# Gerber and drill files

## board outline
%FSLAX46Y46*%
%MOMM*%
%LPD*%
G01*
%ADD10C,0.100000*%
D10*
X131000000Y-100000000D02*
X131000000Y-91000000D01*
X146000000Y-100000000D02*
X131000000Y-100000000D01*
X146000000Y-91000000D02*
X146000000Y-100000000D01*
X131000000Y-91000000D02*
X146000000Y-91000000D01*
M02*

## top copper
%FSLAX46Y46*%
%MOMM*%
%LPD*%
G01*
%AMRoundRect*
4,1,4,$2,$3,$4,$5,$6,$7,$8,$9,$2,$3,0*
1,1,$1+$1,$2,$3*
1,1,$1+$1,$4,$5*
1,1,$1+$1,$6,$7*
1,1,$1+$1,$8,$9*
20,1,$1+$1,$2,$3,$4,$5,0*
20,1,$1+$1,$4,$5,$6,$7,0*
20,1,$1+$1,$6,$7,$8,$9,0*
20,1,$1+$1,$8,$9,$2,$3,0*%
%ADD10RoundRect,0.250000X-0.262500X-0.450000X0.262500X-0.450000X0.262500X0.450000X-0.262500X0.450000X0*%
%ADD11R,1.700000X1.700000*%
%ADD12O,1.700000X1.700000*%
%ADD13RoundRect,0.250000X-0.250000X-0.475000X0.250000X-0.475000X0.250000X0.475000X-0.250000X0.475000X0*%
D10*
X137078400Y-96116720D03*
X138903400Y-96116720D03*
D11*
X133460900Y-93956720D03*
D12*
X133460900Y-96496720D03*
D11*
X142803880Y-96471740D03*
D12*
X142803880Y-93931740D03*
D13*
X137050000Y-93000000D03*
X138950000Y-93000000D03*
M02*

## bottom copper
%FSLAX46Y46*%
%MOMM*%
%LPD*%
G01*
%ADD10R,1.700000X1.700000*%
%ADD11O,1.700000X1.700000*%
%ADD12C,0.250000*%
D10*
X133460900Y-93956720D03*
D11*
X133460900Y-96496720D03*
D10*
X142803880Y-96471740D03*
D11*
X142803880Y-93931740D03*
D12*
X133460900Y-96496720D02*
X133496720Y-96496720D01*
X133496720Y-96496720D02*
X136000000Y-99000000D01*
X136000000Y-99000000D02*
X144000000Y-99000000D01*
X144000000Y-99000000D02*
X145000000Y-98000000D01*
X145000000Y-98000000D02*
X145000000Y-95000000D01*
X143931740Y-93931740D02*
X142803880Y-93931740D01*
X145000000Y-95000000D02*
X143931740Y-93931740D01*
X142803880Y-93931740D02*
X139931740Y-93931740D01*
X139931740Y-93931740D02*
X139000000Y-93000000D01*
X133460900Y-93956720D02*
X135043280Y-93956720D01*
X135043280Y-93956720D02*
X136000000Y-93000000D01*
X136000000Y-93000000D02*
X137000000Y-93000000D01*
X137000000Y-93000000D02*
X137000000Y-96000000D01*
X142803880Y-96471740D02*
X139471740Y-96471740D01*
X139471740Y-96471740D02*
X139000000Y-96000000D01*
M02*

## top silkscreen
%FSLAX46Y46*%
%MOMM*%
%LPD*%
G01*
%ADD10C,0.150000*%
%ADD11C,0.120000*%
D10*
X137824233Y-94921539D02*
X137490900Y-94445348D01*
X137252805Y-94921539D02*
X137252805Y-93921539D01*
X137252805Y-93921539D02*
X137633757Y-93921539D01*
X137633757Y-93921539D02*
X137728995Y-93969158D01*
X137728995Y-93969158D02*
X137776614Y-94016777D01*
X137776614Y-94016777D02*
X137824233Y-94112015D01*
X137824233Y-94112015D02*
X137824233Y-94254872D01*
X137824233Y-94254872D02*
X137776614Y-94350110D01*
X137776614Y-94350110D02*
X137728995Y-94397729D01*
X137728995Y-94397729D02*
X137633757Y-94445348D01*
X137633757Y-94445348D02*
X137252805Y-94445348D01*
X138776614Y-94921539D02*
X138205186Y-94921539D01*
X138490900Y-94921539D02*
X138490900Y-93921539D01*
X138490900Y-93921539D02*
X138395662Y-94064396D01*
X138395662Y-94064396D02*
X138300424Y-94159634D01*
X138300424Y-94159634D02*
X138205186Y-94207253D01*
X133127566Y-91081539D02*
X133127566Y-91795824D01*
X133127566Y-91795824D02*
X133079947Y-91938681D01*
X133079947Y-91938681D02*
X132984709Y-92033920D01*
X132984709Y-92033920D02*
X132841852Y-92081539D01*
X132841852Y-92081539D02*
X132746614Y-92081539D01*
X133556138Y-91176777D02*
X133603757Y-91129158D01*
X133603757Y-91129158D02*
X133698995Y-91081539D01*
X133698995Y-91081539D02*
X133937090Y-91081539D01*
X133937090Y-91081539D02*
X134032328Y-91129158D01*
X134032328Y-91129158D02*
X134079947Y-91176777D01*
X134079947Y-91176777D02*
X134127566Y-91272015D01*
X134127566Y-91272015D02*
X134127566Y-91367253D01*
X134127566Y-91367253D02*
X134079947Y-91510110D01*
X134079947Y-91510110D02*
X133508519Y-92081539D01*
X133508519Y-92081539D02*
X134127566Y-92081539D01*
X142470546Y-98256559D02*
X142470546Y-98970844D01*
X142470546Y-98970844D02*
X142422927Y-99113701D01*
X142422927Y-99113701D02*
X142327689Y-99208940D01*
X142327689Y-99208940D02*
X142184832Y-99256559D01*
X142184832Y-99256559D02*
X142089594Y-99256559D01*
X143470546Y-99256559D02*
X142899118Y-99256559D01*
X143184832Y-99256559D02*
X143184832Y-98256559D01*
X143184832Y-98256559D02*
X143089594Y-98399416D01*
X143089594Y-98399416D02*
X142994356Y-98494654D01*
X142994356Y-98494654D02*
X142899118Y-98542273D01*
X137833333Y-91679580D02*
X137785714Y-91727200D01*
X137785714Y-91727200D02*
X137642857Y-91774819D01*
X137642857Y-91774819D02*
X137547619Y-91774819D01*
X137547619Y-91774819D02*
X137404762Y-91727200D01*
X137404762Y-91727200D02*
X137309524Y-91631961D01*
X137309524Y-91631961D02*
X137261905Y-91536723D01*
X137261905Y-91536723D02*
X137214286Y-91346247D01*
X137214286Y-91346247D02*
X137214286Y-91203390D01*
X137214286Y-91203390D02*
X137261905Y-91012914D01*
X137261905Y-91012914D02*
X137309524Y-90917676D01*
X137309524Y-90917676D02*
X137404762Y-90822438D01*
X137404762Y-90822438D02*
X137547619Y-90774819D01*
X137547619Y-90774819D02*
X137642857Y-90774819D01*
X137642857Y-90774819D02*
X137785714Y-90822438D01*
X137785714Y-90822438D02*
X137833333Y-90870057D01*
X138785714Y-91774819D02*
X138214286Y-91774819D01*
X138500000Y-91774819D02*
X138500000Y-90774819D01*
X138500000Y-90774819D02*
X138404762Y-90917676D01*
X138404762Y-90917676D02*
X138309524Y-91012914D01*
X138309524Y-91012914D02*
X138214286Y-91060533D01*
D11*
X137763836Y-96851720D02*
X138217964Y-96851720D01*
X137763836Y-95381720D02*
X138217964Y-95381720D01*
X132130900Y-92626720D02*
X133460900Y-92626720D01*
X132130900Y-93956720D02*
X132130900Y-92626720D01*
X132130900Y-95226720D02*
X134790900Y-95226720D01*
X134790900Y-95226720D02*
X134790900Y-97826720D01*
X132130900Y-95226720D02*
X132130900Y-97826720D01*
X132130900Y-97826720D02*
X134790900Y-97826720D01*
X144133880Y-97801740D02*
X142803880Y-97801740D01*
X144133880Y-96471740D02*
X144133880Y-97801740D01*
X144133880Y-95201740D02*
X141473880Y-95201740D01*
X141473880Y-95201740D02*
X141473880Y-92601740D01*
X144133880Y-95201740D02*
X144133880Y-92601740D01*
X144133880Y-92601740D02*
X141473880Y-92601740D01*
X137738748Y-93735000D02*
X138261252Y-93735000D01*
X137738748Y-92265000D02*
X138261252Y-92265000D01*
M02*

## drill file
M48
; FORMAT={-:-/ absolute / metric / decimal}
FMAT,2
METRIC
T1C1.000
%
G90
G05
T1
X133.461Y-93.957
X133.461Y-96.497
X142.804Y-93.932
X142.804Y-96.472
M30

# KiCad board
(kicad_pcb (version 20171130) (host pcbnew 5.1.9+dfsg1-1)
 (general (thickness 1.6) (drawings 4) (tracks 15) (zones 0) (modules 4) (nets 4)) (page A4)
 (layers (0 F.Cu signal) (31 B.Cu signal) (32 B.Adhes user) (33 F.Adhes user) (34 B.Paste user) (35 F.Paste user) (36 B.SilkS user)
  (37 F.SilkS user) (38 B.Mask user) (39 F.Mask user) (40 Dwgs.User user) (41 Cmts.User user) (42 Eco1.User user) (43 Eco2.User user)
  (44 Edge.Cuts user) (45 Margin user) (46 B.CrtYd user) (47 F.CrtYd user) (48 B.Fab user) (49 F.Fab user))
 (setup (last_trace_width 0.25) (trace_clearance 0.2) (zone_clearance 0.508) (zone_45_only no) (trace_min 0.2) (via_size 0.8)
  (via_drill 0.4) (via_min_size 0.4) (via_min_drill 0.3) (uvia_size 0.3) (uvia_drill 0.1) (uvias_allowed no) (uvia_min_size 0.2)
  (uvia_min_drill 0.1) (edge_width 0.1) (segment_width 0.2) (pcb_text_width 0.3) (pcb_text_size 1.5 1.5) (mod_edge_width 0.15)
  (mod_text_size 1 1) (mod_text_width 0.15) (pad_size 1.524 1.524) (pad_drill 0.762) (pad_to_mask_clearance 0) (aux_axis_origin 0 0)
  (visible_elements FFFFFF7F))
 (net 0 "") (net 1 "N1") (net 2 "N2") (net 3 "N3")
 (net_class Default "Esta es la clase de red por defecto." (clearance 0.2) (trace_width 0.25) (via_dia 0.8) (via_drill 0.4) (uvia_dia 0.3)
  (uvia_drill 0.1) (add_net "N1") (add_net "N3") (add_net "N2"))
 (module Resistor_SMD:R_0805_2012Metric (layer F.Cu) (at 137.9909 96.11672)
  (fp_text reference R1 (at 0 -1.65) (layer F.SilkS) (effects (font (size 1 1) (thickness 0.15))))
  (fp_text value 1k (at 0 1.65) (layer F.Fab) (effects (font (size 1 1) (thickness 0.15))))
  (fp_line (start -0.227064 0.735) (end 0.227064 0.735) (layer F.SilkS) (width 0.12))
  (fp_line (start -0.227064 -0.735) (end 0.227064 -0.735) (layer F.SilkS) (width 0.12))
  (pad 1 smd roundrect (at -0.9125 0) (size 1.025 1.4) (layers F.Cu F.Paste F.Mask) (roundrect_rratio 0.243902) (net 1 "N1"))
  (pad 2 smd roundrect (at 0.9125 0) (size 1.025 1.4) (layers F.Cu F.Paste F.Mask) (roundrect_rratio 0.243902) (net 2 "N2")))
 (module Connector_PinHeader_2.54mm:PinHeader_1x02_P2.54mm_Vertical (layer F.Cu) (at 133.4609 93.95672)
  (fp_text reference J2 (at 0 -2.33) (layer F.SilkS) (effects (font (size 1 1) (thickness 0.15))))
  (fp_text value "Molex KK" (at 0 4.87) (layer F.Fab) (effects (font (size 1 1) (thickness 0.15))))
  (fp_line (start -1.33 -1.33) (end 0 -1.33) (layer F.SilkS) (width 0.12))
  (fp_line (start -1.33 0) (end -1.33 -1.33) (layer F.SilkS) (width 0.12))
  (fp_line (start -1.33 1.27) (end 1.33 1.27) (layer F.SilkS) (width 0.12))
  (fp_line (start 1.33 1.27) (end 1.33 3.87) (layer F.SilkS) (width 0.12))
  (fp_line (start -1.33 1.27) (end -1.33 3.87) (layer F.SilkS) (width 0.12))
  (fp_line (start -1.33 3.87) (end 1.33 3.87) (layer F.SilkS) (width 0.12))
  (pad 1 thru_hole rect (at 0 0) (size 1.7 1.7) (drill 1) (layers *.Cu *.Mask) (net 1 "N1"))
  (pad 2 thru_hole oval (at 0 2.54) (size 1.7 1.7) (drill 1) (layers *.Cu *.Mask) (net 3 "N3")))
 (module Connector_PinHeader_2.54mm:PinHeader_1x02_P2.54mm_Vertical (layer F.Cu) (at 142.80388 96.47174 180)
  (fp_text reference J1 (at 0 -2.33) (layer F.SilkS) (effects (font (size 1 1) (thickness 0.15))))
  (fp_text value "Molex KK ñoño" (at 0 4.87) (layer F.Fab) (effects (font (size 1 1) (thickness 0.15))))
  (fp_line (start -1.33 -1.33) (end 0 -1.33) (layer F.SilkS) (width 0.12))
  (fp_line (start -1.33 0) (end -1.33 -1.33) (layer F.SilkS) (width 0.12))
  (fp_line (start -1.33 1.27) (end 1.33 1.27) (layer F.SilkS) (width 0.12))
  (fp_line (start 1.33 1.27) (end 1.33 3.87) (layer F.SilkS) (width 0.12))
  (fp_line (start -1.33 1.27) (end -1.33 3.87) (layer F.SilkS) (width 0.12))
  (fp_line (start -1.33 3.87) (end 1.33 3.87) (layer F.SilkS) (width 0.12))
  (pad 1 thru_hole rect (at 0 0 180) (size 1.7 1.7) (drill 1) (layers *.Cu *.Mask) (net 2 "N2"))
  (pad 2 thru_hole oval (at 0 2.54 180) (size 1.7 1.7) (drill 1) (layers *.Cu *.Mask) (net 3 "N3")))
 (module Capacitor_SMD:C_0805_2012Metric (layer F.Cu) (at 138 93)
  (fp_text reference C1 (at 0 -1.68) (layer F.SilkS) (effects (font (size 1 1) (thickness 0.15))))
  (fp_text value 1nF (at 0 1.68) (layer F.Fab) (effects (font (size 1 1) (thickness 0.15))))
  (fp_line (start -0.261252 0.735) (end 0.261252 0.735) (layer F.SilkS) (width 0.12))
  (fp_line (start -0.261252 -0.735) (end 0.261252 -0.735) (layer F.SilkS) (width 0.12))
  (pad 1 smd roundrect (at -0.95 0) (size 1 1.45) (layers F.Cu F.Paste F.Mask) (roundrect_rratio 0.25) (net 1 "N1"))
  (pad 2 smd roundrect (at 0.95 0) (size 1 1.45) (layers F.Cu F.Paste F.Mask) (roundrect_rratio 0.25) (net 3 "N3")))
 (gr_line (start 131 100) (end 131 91) (layer Edge.Cuts) (width 0.1))
 (gr_line (start 146 100) (end 131 100) (layer Edge.Cuts) (width 0.1))
 (gr_line (start 146 91) (end 146 100) (layer Edge.Cuts) (width 0.1))
 (gr_line (start 131 91) (end 146 91) (layer Edge.Cuts) (width 0.1))
 (segment (start 133.4609 96.49672) (end 133.49672 96.49672) (width 0.25) (layer B.Cu) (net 3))
 (segment (start 133.49672 96.49672) (end 136 99) (width 0.25) (layer B.Cu) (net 3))
 (segment (start 136 99) (end 144 99) (width 0.25) (layer B.Cu) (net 3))
 (segment (start 144 99) (end 145 98) (width 0.25) (layer B.Cu) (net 3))
 (segment (start 145 98) (end 145 95) (width 0.25) (layer B.Cu) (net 3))
 (segment (start 143.93174 93.93174) (end 142.80388 93.93174) (width 0.25) (layer B.Cu) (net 3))
 (segment (start 145 95) (end 143.93174 93.93174) (width 0.25) (layer B.Cu) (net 3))
 (segment (start 142.80388 93.93174) (end 139.93174 93.93174) (width 0.25) (layer B.Cu) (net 3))
 (segment (start 139.93174 93.93174) (end 139 93) (width 0.25) (layer B.Cu) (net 3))
 (segment (start 133.4609 93.95672) (end 135.04328 93.95672) (width 0.25) (layer B.Cu) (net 1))
 (segment (start 135.04328 93.95672) (end 136 93) (width 0.25) (layer B.Cu) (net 1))
 (segment (start 136 93) (end 137 93) (width 0.25) (layer B.Cu) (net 1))
 (segment (start 137 93) (end 137 96) (width 0.25) (layer B.Cu) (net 1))
 (segment (start 142.80388 96.47174) (end 139.47174 96.47174) (width 0.25) (layer B.Cu) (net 2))
 (segment (start 139.47174 96.47174) (end 139 96) (width 0.25) (layer B.Cu) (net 2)))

